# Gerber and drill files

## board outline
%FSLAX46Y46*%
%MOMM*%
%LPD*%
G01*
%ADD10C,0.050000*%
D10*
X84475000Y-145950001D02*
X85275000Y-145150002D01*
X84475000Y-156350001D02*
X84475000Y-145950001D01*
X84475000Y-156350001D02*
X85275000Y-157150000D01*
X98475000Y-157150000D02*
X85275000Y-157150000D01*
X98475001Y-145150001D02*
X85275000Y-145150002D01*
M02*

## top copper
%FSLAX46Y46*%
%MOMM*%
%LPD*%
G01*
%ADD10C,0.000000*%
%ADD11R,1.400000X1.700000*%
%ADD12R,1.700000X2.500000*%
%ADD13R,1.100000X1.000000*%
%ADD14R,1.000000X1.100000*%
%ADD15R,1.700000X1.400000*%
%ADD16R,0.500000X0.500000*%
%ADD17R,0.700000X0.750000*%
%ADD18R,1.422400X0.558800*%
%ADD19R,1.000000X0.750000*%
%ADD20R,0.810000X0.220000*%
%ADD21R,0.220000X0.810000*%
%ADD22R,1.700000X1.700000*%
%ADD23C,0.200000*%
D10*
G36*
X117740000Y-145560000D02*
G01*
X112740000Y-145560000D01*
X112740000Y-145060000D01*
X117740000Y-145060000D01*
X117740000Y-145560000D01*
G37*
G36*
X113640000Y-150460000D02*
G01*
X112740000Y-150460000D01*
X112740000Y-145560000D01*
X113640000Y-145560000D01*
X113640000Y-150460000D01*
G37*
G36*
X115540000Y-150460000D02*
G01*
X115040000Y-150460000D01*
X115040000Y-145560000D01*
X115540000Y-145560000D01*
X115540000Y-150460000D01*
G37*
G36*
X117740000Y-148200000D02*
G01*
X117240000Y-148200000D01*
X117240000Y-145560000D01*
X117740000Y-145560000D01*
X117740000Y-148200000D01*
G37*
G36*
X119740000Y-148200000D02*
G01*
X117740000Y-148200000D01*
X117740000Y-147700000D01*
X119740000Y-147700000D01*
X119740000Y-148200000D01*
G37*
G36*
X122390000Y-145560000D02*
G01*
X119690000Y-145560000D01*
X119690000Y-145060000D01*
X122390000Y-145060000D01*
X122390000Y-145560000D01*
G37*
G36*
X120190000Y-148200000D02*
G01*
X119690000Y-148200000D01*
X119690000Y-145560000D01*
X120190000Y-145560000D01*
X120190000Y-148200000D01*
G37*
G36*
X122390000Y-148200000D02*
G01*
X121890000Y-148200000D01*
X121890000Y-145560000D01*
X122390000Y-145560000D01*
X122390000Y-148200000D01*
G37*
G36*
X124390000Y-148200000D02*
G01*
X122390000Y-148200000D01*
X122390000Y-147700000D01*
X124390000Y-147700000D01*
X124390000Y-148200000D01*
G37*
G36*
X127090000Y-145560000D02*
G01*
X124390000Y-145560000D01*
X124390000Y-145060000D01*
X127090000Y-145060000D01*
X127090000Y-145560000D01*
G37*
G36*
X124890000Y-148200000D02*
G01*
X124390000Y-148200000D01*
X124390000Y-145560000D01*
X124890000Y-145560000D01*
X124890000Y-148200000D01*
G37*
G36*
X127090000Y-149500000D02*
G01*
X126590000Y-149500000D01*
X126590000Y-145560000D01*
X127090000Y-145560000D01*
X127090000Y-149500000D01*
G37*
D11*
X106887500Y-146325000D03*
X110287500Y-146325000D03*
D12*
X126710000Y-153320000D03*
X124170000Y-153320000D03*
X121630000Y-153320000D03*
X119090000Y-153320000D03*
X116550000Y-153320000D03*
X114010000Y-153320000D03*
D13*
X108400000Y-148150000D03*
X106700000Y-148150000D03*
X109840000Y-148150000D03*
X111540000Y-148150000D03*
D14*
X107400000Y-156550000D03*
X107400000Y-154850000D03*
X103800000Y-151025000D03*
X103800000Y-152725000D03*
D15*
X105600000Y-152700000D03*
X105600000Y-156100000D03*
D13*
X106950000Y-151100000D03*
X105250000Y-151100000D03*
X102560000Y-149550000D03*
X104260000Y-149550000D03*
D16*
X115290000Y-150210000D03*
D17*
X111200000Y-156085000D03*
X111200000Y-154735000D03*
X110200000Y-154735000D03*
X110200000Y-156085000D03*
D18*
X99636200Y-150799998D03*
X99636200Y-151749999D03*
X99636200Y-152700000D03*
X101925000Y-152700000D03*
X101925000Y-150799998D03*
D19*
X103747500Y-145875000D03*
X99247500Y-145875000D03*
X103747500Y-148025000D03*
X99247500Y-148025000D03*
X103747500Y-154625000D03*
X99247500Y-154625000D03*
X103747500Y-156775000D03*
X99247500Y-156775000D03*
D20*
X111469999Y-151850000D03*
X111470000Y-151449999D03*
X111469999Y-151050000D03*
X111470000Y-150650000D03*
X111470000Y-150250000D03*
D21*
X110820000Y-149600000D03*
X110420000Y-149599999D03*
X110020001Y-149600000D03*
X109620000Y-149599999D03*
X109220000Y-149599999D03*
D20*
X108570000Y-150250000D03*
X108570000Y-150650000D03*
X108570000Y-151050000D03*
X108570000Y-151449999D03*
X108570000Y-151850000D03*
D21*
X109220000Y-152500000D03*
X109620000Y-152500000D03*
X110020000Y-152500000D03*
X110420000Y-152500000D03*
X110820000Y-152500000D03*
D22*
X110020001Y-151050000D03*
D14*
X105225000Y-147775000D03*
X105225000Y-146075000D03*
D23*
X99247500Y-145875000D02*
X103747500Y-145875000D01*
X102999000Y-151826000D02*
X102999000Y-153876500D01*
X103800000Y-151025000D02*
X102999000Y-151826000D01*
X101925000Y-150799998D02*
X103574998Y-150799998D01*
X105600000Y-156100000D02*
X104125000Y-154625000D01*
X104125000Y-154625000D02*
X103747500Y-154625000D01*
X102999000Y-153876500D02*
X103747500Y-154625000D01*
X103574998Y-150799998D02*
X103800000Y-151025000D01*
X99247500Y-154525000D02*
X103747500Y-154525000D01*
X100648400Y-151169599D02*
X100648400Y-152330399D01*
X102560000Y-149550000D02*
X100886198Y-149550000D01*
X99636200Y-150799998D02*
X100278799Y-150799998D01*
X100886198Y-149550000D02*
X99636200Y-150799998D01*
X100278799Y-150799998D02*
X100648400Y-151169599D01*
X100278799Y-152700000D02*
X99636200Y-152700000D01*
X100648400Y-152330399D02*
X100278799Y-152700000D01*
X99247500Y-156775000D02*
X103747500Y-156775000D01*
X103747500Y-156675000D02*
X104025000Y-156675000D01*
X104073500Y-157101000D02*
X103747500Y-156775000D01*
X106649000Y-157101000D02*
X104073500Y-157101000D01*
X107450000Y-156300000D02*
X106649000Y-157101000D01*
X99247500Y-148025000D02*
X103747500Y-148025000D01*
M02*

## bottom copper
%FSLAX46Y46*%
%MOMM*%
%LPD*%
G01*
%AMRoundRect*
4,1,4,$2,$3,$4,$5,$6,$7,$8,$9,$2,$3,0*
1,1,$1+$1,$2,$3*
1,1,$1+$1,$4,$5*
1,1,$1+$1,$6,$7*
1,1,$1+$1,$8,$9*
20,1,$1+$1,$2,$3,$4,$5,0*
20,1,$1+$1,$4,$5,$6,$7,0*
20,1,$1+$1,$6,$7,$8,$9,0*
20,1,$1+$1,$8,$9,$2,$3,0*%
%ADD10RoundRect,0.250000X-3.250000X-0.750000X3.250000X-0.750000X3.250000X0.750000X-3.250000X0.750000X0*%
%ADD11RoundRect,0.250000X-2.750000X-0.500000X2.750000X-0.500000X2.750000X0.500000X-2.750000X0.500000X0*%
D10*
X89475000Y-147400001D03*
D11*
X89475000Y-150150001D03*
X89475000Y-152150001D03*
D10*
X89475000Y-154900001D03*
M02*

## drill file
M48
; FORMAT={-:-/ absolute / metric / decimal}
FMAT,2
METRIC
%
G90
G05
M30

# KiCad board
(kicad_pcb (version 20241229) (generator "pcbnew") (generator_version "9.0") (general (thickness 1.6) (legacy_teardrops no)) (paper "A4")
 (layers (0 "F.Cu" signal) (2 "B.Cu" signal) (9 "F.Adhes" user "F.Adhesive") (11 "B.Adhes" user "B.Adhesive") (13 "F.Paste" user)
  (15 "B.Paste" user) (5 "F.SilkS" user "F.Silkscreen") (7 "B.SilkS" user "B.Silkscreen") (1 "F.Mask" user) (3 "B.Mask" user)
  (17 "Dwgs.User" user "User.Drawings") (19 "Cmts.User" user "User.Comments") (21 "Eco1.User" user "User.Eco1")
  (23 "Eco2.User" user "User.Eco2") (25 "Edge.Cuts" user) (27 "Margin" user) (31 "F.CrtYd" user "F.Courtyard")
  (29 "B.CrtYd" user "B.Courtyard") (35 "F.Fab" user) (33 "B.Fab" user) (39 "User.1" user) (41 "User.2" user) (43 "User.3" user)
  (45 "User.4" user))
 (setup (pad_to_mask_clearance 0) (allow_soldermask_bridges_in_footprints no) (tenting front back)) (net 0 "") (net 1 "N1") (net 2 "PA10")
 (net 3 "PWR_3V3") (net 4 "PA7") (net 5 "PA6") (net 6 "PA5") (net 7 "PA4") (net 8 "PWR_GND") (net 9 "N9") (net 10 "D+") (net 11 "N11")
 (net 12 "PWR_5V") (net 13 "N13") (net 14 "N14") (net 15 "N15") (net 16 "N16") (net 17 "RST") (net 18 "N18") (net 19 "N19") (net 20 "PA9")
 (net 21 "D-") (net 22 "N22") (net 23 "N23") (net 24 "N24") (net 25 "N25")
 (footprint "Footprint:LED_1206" (layer "F.Cu") (at 108.5875 146.325)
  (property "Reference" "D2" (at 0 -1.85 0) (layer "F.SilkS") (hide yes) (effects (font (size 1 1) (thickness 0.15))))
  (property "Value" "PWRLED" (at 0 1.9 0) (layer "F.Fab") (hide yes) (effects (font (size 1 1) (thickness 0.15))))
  (pad "1" smd rect (at -1.7 0) (size 1.4 1.7) (layers "F.Cu" "F.Mask" "F.Paste") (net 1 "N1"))
  (pad "2" smd rect (at 1.7 0) (size 1.4 1.7) (layers "F.Cu" "F.Mask" "F.Paste") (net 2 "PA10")))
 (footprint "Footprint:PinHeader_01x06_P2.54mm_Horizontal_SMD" (layer "F.Cu") (at 126.71 153.32 -90)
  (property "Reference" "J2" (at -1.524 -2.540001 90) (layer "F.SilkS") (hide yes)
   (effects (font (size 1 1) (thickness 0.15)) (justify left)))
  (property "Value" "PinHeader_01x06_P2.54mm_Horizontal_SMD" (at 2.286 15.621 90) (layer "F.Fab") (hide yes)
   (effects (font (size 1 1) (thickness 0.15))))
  (pad "1" smd rect (at 0 0 270) (size 2.5 1.7) (layers "F.Cu" "F.Mask" "F.Paste") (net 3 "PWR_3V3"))
  (pad "2" smd rect (at 0 2.54 270) (size 2.5 1.7) (layers "F.Cu" "F.Mask" "F.Paste") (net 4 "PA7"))
  (pad "3" smd rect (at 0 5.08 270) (size 2.5 1.7) (layers "F.Cu" "F.Mask" "F.Paste") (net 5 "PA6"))
  (pad "4" smd rect (at 0 7.62 270) (size 2.5 1.7) (layers "F.Cu" "F.Mask" "F.Paste") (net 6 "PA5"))
  (pad "5" smd rect (at 0 10.16 270) (size 2.5 1.7) (layers "F.Cu" "F.Mask" "F.Paste") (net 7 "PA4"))
  (pad "6" smd rect (at 0 12.7 270) (size 2.5 1.7) (layers "F.Cu" "F.Mask" "F.Paste") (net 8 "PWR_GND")))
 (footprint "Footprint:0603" (layer "F.Cu") (at 107.55 148.15 180)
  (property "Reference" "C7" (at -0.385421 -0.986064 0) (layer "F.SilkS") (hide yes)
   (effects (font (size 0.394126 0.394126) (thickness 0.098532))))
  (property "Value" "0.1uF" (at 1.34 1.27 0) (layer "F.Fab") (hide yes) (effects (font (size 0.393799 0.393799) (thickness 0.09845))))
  (pad "1" smd rect (at -0.85 0 180) (size 1.1 1) (layers "F.Cu" "F.Mask" "F.Paste") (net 3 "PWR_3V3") (solder_mask_margin 0.102))
  (pad "2" smd rect (at 0.85 0 180) (size 1.1 1) (layers "F.Cu" "F.Mask" "F.Paste") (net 8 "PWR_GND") (solder_mask_margin 0.102)))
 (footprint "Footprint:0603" (layer "F.Cu") (at 110.69 148.15)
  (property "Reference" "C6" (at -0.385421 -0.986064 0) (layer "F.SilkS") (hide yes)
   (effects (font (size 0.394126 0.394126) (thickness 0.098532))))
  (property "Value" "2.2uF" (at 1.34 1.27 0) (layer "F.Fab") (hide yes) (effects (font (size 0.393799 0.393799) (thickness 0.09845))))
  (pad "1" smd rect (at -0.85 0) (size 1.1 1) (layers "F.Cu" "F.Mask" "F.Paste") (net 3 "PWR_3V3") (solder_mask_margin 0.102))
  (pad "2" smd rect (at 0.85 0) (size 1.1 1) (layers "F.Cu" "F.Mask" "F.Paste") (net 8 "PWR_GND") (solder_mask_margin 0.102)))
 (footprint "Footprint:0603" (layer "F.Cu") (at 107.4 155.7 90)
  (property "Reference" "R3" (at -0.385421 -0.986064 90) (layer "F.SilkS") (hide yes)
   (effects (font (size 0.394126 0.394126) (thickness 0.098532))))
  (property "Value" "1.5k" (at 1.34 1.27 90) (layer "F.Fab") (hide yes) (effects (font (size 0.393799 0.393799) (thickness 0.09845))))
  (pad "1" smd rect (at -0.85 0 90) (size 1.1 1) (layers "F.Cu" "F.Mask" "F.Paste") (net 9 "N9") (solder_mask_margin 0.102))
  (pad "2" smd rect (at 0.85 0 90) (size 1.1 1) (layers "F.Cu" "F.Mask" "F.Paste") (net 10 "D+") (solder_mask_margin 0.102)))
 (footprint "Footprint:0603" (layer "F.Cu") (at 103.8 151.875 -90)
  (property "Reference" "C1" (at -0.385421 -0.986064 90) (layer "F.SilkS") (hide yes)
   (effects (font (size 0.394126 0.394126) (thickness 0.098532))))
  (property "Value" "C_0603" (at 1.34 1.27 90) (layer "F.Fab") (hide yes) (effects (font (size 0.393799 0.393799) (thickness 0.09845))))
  (pad "1" smd rect (at -0.85 0 270) (size 1.1 1) (layers "F.Cu" "F.Mask" "F.Paste") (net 3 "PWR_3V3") (solder_mask_margin 0.102))
  (pad "2" smd rect (at 0.85 0 270) (size 1.1 1) (layers "F.Cu" "F.Mask" "F.Paste") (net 8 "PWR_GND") (solder_mask_margin 0.102)))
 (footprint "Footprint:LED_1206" (layer "F.Cu") (at 105.6 154.4 -90)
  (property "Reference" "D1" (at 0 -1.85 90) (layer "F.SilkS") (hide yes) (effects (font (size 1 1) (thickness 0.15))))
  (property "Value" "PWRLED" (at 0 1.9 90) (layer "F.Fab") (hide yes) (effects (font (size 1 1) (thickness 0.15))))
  (pad "1" smd rect (at -1.7 0 270) (size 1.4 1.7) (layers "F.Cu" "F.Mask" "F.Paste") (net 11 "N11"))
  (pad "2" smd rect (at 1.7 0 270) (size 1.4 1.7) (layers "F.Cu" "F.Mask" "F.Paste") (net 3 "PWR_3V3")))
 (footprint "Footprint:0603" (layer "F.Cu") (at 106.1 151.1 180)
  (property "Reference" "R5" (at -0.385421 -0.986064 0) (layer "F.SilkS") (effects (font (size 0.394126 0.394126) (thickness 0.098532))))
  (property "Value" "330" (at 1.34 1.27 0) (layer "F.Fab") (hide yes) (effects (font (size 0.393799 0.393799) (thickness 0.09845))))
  (pad "1" smd rect (at -0.85 0 180) (size 1.1 1) (layers "F.Cu" "F.Mask" "F.Paste") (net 8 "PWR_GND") (solder_mask_margin 0.102))
  (pad "2" smd rect (at 0.85 0 180) (size 1.1 1) (layers "F.Cu" "F.Mask" "F.Paste") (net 11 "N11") (solder_mask_margin 0.102)))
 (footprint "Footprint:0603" (layer "F.Cu") (at 103.41 149.55)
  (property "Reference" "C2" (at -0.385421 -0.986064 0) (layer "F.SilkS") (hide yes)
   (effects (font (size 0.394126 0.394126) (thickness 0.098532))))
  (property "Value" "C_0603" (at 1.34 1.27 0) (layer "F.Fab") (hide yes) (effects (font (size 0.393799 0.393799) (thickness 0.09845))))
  (pad "1" smd rect (at -0.85 0) (size 1.1 1) (layers "F.Cu" "F.Mask" "F.Paste") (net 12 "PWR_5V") (solder_mask_margin 0.102))
  (pad "2" smd rect (at 0.85 0) (size 1.1 1) (layers "F.Cu" "F.Mask" "F.Paste") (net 8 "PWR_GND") (solder_mask_margin 0.102)))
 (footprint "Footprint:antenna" (layer "F.Cu") (at 112.74 149.96)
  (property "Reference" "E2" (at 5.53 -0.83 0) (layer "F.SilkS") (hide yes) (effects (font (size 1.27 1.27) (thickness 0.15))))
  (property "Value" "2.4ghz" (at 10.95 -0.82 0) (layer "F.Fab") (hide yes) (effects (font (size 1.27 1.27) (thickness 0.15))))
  (fp_poly (pts (xy 0 -4.9) (xy 0 -4.4) (xy 5 -4.4) (xy 5 -4.9) (xy 0 -4.9)) (stroke (width 0) (type solid)) (fill yes) (layer "F.Cu"))
  (fp_poly (pts (xy 0 -4.4) (xy 0 0.5) (xy 0.9 0.5) (xy 0.9 -4.4) (xy 0 -4.4)) (stroke (width 0) (type solid)) (fill yes) (layer "F.Cu"))
  (fp_poly
   (pts (xy 2.3 -4.4) (xy 2.3 0.5) (xy 2.8 0.5) (xy 2.8 -4.4) (xy 2.3 -4.4)) (stroke (width 0) (type solid)) (fill yes) (layer "F.Cu"))
  (fp_poly
   (pts (xy 4.5 -4.4) (xy 4.5 -1.76) (xy 5 -1.76) (xy 5 -4.4) (xy 4.5 -4.4)) (stroke (width 0) (type solid)) (fill yes) (layer "F.Cu"))
  (fp_poly (pts (xy 5 -2.26) (xy 5 -1.76) (xy 7 -1.76) (xy 7 -2.26) (xy 5 -2.26)) (stroke (width 0) (type solid)) (fill yes) (layer "F.Cu"))
  (fp_poly
   (pts (xy 6.95 -4.9) (xy 6.95 -4.4) (xy 9.65 -4.4) (xy 9.65 -4.9) (xy 6.95 -4.9)) (stroke (width 0) (type solid)) (fill yes)
   (layer "F.Cu"))
  (fp_poly
   (pts (xy 6.95 -4.4) (xy 6.95 -1.76) (xy 7.45 -1.76) (xy 7.45 -4.4) (xy 6.95 -4.4)) (stroke (width 0) (type solid)) (fill yes)
   (layer "F.Cu"))
  (fp_poly
   (pts (xy 9.15 -4.4) (xy 9.15 -1.76) (xy 9.65 -1.76) (xy 9.65 -4.4) (xy 9.15 -4.4)) (stroke (width 0) (type solid)) (fill yes)
   (layer "F.Cu"))
  (fp_poly
   (pts (xy 9.65 -2.26) (xy 9.65 -1.76) (xy 11.65 -1.76) (xy 11.65 -2.26) (xy 9.65 -2.26)) (stroke (width 0) (type solid)) (fill yes)
   (layer "F.Cu"))
  (fp_poly
   (pts (xy 11.65 -4.9) (xy 11.65 -4.4) (xy 14.35 -4.4) (xy 14.35 -4.9) (xy 11.65 -4.9)) (stroke (width 0) (type solid)) (fill yes)
   (layer "F.Cu"))
  (fp_poly
   (pts (xy 11.65 -4.4) (xy 11.65 -1.76) (xy 12.15 -1.76) (xy 12.15 -4.4) (xy 11.65 -4.4)) (stroke (width 0) (type solid)) (fill yes)
   (layer "F.Cu"))
  (fp_poly
   (pts (xy 13.85 -4.4) (xy 13.85 -0.46) (xy 14.35 -0.46) (xy 14.35 -4.4) (xy 13.85 -4.4)) (stroke (width 0) (type solid)) (fill yes)
   (layer "F.Cu"))
  (pad "1" smd rect (at 2.55 0.25) (size 0.5 0.5) (layers "F.Cu" "F.Mask" "F.Paste") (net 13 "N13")))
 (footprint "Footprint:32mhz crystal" (layer "F.Cu") (at 110.7 155.41 180)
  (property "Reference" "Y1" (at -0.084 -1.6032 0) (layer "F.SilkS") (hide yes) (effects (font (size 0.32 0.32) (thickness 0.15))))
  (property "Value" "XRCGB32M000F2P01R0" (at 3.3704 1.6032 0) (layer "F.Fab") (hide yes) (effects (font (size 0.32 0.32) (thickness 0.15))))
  (pad "1" smd rect (at -0.5 -0.675 180) (size 0.7 0.75) (layers "F.Cu" "F.Mask" "F.Paste") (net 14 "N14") (solder_mask_margin 0.102))
  (pad "2" smd rect (at -0.5 0.675 180) (size 0.7 0.75) (layers "F.Cu" "F.Mask" "F.Paste") (solder_mask_margin 0.102))
  (pad "3" smd rect (at 0.5 0.675 180) (size 0.7 0.75) (layers "F.Cu" "F.Mask" "F.Paste") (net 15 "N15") (solder_mask_margin 0.102))
  (pad "4" smd rect (at 0.5 -0.675 180) (size 0.7 0.75) (layers "F.Cu" "F.Mask" "F.Paste") (solder_mask_margin 0.102)))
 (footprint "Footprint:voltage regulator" (layer "F.Cu") (at 100.7806 151.749999)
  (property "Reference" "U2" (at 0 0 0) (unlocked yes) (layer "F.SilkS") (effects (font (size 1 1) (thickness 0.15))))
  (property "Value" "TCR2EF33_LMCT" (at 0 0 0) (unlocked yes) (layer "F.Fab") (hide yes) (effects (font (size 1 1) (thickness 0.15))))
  (pad "1" smd rect (at -1.1444 -0.950001) (size 1.4224 0.5588) (layers "F.Cu" "F.Mask" "F.Paste") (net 12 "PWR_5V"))
  (pad "2" smd rect (at -1.1444 0) (size 1.4224 0.5588) (layers "F.Cu" "F.Mask" "F.Paste") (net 8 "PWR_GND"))
  (pad "3" smd rect (at -1.1444 0.950001) (size 1.4224 0.5588) (layers "F.Cu" "F.Mask" "F.Paste") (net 12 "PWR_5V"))
  (pad "4" smd rect (at 1.1444 0.950001) (size 1.4224 0.5588) (layers "F.Cu" "F.Mask" "F.Paste") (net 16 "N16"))
  (pad "5" smd rect (at 1.1444 -0.950001) (size 1.4224 0.5588) (layers "F.Cu" "F.Mask" "F.Paste") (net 3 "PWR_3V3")))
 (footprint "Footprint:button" (layer "F.Cu") (at 101.4975 146.95 180)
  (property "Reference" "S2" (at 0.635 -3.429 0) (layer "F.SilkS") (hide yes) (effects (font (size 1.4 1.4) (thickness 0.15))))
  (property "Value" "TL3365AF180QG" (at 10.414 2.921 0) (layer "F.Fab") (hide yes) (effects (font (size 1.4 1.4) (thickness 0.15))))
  (pad "1" smd rect (at -2.25 1.075 180) (size 1 0.75) (layers "F.Cu" "F.Mask" "F.Paste") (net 8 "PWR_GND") (solder_mask_margin 0.102))
  (pad "2" smd rect (at 2.25 1.075 180) (size 1 0.75) (layers "F.Cu" "F.Mask" "F.Paste") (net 8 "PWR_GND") (solder_mask_margin 0.102))
  (pad "3" smd rect (at -2.25 -1.075 180) (size 1 0.75) (layers "F.Cu" "F.Mask" "F.Paste") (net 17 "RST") (solder_mask_margin 0.102))
  (pad "4" smd rect (at 2.25 -1.075 180) (size 1 0.75) (layers "F.Cu" "F.Mask" "F.Paste") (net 17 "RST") (solder_mask_margin 0.102)))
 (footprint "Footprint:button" (layer "F.Cu") (at 101.4975 155.7 180)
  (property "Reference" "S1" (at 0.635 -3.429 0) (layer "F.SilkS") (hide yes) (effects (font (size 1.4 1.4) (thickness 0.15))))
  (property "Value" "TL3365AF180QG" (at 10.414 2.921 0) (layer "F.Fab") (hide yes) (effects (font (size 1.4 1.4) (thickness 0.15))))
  (pad "1" smd rect (at -2.25 1.075 180) (size 1 0.75) (layers "F.Cu" "F.Mask" "F.Paste") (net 3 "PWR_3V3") (solder_mask_margin 0.102))
  (pad "2" smd rect (at 2.25 1.075 180) (size 1 0.75) (layers "F.Cu" "F.Mask" "F.Paste") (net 3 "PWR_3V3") (solder_mask_margin 0.102))
  (pad "3" smd rect (at -2.25 -1.075 180) (size 1 0.75) (layers "F.Cu" "F.Mask" "F.Paste") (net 9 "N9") (solder_mask_margin 0.102))
  (pad "4" smd rect (at 2.25 -1.075 180) (size 1 0.75) (layers "F.Cu" "F.Mask" "F.Paste") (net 9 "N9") (solder_mask_margin 0.102)))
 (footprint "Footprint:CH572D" (layer "F.Cu") (at 109.25 148.99 180)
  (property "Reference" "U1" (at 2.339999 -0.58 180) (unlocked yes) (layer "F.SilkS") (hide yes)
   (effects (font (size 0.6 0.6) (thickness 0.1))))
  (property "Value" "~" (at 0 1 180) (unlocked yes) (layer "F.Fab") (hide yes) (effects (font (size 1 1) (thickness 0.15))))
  (pad "1" smd rect (at -2.219999 -2.86 180) (size 0.81 0.22) (layers "F.Cu" "F.Paste") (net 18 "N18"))
  (pad "2" smd rect (at -2.22 -2.459999 180) (size 0.81 0.22) (layers "F.Cu" "F.Paste") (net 14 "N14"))
  (pad "3" smd rect (at -2.219999 -2.06 180) (size 0.81 0.22) (layers "F.Cu" "F.Paste") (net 15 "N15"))
  (pad "4" smd rect (at -2.22 -1.66 180) (size 0.81 0.22) (layers "F.Cu" "F.Paste") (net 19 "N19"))
  (pad "5" smd rect (at -2.22 -1.26 180) (size 0.81 0.22) (layers "F.Cu" "F.Paste") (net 13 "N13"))
  (pad "6" smd rect (at -1.57 -0.61 180) (size 0.22 0.81) (layers "F.Cu" "F.Paste") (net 3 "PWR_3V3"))
  (pad "7" smd rect (at -1.17 -0.609999 180) (size 0.22 0.81) (layers "F.Cu" "F.Paste") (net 3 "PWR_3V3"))
  (pad "8" smd rect (at -0.770001 -0.61 180) (size 0.22 0.81) (layers "F.Cu" "F.Paste") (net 12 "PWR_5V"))
  (pad "9" smd rect (at -0.37 -0.609999 180) (size 0.22 0.81) (layers "F.Cu" "F.Paste") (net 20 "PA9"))
  (pad "10" smd rect (at 0.03 -0.609999 180) (size 0.22 0.81) (layers "F.Cu" "F.Paste") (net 17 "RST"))
  (pad "11" smd rect (at 0.68 -1.26 180) (size 0.81 0.22) (layers "F.Cu" "F.Paste") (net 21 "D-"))
  (pad "12" smd rect (at 0.68 -1.66 180) (size 0.81 0.22) (layers "F.Cu" "F.Paste") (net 10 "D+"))
  (pad "13" smd rect (at 0.68 -2.06 180) (size 0.81 0.22) (layers "F.Cu" "F.Paste") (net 7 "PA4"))
  (pad "14" smd rect (at 0.68 -2.459999 180) (size 0.81 0.22) (layers "F.Cu" "F.Paste") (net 6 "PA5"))
  (pad "15" smd rect (at 0.68 -2.86 180) (size 0.81 0.22) (layers "F.Cu" "F.Paste") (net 5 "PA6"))
  (pad "16" smd rect (at 0.03 -3.51 180) (size 0.22 0.81) (layers "F.Cu" "F.Paste") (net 4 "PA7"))
  (pad "17" smd rect (at -0.37 -3.51 180) (size 0.22 0.81) (layers "F.Cu" "F.Paste") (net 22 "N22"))
  (pad "18" smd rect (at -0.77 -3.51 180) (size 0.22 0.81) (layers "F.Cu" "F.Paste") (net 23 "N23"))
  (pad "19" smd rect (at -1.17 -3.51 180) (size 0.22 0.81) (layers "F.Cu" "F.Paste") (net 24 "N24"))
  (pad "20" smd rect (at -1.57 -3.51 180) (size 0.22 0.81) (layers "F.Cu" "F.Paste") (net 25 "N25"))
  (pad "21" smd rect (at -0.770001 -2.06 180) (size 1.7 1.7) (layers "F.Cu") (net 8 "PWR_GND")))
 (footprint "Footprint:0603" (layer "F.Cu") (at 105.225 146.925 90)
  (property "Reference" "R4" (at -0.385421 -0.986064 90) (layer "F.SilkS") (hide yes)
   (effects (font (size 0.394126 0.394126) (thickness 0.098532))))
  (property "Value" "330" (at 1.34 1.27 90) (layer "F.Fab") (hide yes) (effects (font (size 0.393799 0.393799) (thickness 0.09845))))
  (pad "1" smd rect (at -0.85 0 90) (size 1.1 1) (layers "F.Cu" "F.Mask" "F.Paste") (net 8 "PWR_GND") (solder_mask_margin 0.102))
  (pad "2" smd rect (at 0.85 0 90) (size 1.1 1) (layers "F.Cu" "F.Mask" "F.Paste") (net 1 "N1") (solder_mask_margin 0.102)))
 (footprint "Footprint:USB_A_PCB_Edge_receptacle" (layer "B.Cu") (at 89.475 151.150001)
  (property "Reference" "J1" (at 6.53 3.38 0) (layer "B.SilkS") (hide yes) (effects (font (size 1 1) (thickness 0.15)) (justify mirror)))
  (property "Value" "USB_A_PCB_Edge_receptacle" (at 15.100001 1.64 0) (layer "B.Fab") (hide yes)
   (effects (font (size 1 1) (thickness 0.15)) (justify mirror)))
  (fp_line (start -5 -5.2) (end -4.2 -5.999999) (stroke (width 0.05) (type default)) (layer "Edge.Cuts"))
  (fp_line (start -5 5.2) (end -5 -5.2) (stroke (width 0.05) (type default)) (layer "Edge.Cuts"))
  (fp_line (start -5 5.2) (end -4.2 5.999999) (stroke (width 0.05) (type default)) (layer "Edge.Cuts"))
  (fp_line (start 9 5.999999) (end -4.2 5.999999) (stroke (width 0.05) (type default)) (layer "Edge.Cuts"))
  (fp_line (start 9.000001 -6) (end -4.2 -5.999999) (stroke (width 0.05) (type default)) (layer "Edge.Cuts"))
  (pad "1" smd roundrect (at 0 -3.75) (size 7 2) (layers "B.Cu" "B.Mask") (roundrect_rratio 0.125) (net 12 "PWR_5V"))
  (pad "2" smd roundrect (at 0 -1) (size 6 1.5) (layers "B.Cu" "B.Mask") (roundrect_rratio 0.1666666667) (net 21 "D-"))
  (pad "3" smd roundrect (at 0 1) (size 6 1.5) (layers "B.Cu" "B.Mask") (roundrect_rratio 0.1666666667) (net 10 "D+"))
  (pad "4" smd roundrect (at 0 3.75) (size 7 2) (layers "B.Cu" "B.Mask") (roundrect_rratio 0.125) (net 8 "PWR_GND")))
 (segment (start 99.2475 145.875) (end 103.7475 145.875) (width 0.2) (layer "F.Cu") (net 8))
 (segment (start 102.999 151.826) (end 102.999 153.8765) (width 0.2) (layer "F.Cu") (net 3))
 (segment (start 103.8 151.025) (end 102.999 151.826) (width 0.2) (layer "F.Cu") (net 3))
 (segment (start 101.925 150.799998) (end 103.574998 150.799998) (width 0.2) (layer "F.Cu") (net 3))
 (segment (start 105.6 156.1) (end 104.125 154.625) (width 0.2) (layer "F.Cu") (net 3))
 (segment (start 104.125 154.625) (end 103.7475 154.625) (width 0.2) (layer "F.Cu") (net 3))
 (segment (start 102.999 153.8765) (end 103.7475 154.625) (width 0.2) (layer "F.Cu") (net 3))
 (segment (start 103.574998 150.799998) (end 103.8 151.025) (width 0.2) (layer "F.Cu") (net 3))
 (segment (start 99.2475 154.525) (end 103.7475 154.525) (width 0.2) (layer "F.Cu") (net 3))
 (segment (start 100.6484 151.169599) (end 100.6484 152.330399) (width 0.2) (layer "F.Cu") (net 12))
 (segment (start 102.56 149.55) (end 100.886198 149.55) (width 0.2) (layer "F.Cu") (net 12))
 (segment (start 99.6362 150.799998) (end 100.278799 150.799998) (width 0.2) (layer "F.Cu") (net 12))
 (segment (start 100.886198 149.55) (end 99.6362 150.799998) (width 0.2) (layer "F.Cu") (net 12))
 (segment (start 100.278799 150.799998) (end 100.6484 151.169599) (width 0.2) (layer "F.Cu") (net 12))
 (segment (start 100.278799 152.7) (end 99.6362 152.7) (width 0.2) (layer "F.Cu") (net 12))
 (segment (start 100.6484 152.330399) (end 100.278799 152.7) (width 0.2) (layer "F.Cu") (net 12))
 (segment (start 99.2475 156.775) (end 103.7475 156.775) (width 0.2) (layer "F.Cu") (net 9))
 (segment (start 103.7475 156.675) (end 104.025 156.675) (width 0.2) (layer "F.Cu") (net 9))
 (segment (start 104.0735 157.101) (end 103.7475 156.775) (width 0.2) (layer "F.Cu") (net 9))
 (segment (start 106.649 157.101) (end 104.0735 157.101) (width 0.2) (layer "F.Cu") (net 9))
 (segment (start 107.45 156.3) (end 106.649 157.101) (width 0.2) (layer "F.Cu") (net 9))
 (segment (start 99.2475 148.025) (end 103.7475 148.025) (width 0.2) (layer "F.Cu") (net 17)))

